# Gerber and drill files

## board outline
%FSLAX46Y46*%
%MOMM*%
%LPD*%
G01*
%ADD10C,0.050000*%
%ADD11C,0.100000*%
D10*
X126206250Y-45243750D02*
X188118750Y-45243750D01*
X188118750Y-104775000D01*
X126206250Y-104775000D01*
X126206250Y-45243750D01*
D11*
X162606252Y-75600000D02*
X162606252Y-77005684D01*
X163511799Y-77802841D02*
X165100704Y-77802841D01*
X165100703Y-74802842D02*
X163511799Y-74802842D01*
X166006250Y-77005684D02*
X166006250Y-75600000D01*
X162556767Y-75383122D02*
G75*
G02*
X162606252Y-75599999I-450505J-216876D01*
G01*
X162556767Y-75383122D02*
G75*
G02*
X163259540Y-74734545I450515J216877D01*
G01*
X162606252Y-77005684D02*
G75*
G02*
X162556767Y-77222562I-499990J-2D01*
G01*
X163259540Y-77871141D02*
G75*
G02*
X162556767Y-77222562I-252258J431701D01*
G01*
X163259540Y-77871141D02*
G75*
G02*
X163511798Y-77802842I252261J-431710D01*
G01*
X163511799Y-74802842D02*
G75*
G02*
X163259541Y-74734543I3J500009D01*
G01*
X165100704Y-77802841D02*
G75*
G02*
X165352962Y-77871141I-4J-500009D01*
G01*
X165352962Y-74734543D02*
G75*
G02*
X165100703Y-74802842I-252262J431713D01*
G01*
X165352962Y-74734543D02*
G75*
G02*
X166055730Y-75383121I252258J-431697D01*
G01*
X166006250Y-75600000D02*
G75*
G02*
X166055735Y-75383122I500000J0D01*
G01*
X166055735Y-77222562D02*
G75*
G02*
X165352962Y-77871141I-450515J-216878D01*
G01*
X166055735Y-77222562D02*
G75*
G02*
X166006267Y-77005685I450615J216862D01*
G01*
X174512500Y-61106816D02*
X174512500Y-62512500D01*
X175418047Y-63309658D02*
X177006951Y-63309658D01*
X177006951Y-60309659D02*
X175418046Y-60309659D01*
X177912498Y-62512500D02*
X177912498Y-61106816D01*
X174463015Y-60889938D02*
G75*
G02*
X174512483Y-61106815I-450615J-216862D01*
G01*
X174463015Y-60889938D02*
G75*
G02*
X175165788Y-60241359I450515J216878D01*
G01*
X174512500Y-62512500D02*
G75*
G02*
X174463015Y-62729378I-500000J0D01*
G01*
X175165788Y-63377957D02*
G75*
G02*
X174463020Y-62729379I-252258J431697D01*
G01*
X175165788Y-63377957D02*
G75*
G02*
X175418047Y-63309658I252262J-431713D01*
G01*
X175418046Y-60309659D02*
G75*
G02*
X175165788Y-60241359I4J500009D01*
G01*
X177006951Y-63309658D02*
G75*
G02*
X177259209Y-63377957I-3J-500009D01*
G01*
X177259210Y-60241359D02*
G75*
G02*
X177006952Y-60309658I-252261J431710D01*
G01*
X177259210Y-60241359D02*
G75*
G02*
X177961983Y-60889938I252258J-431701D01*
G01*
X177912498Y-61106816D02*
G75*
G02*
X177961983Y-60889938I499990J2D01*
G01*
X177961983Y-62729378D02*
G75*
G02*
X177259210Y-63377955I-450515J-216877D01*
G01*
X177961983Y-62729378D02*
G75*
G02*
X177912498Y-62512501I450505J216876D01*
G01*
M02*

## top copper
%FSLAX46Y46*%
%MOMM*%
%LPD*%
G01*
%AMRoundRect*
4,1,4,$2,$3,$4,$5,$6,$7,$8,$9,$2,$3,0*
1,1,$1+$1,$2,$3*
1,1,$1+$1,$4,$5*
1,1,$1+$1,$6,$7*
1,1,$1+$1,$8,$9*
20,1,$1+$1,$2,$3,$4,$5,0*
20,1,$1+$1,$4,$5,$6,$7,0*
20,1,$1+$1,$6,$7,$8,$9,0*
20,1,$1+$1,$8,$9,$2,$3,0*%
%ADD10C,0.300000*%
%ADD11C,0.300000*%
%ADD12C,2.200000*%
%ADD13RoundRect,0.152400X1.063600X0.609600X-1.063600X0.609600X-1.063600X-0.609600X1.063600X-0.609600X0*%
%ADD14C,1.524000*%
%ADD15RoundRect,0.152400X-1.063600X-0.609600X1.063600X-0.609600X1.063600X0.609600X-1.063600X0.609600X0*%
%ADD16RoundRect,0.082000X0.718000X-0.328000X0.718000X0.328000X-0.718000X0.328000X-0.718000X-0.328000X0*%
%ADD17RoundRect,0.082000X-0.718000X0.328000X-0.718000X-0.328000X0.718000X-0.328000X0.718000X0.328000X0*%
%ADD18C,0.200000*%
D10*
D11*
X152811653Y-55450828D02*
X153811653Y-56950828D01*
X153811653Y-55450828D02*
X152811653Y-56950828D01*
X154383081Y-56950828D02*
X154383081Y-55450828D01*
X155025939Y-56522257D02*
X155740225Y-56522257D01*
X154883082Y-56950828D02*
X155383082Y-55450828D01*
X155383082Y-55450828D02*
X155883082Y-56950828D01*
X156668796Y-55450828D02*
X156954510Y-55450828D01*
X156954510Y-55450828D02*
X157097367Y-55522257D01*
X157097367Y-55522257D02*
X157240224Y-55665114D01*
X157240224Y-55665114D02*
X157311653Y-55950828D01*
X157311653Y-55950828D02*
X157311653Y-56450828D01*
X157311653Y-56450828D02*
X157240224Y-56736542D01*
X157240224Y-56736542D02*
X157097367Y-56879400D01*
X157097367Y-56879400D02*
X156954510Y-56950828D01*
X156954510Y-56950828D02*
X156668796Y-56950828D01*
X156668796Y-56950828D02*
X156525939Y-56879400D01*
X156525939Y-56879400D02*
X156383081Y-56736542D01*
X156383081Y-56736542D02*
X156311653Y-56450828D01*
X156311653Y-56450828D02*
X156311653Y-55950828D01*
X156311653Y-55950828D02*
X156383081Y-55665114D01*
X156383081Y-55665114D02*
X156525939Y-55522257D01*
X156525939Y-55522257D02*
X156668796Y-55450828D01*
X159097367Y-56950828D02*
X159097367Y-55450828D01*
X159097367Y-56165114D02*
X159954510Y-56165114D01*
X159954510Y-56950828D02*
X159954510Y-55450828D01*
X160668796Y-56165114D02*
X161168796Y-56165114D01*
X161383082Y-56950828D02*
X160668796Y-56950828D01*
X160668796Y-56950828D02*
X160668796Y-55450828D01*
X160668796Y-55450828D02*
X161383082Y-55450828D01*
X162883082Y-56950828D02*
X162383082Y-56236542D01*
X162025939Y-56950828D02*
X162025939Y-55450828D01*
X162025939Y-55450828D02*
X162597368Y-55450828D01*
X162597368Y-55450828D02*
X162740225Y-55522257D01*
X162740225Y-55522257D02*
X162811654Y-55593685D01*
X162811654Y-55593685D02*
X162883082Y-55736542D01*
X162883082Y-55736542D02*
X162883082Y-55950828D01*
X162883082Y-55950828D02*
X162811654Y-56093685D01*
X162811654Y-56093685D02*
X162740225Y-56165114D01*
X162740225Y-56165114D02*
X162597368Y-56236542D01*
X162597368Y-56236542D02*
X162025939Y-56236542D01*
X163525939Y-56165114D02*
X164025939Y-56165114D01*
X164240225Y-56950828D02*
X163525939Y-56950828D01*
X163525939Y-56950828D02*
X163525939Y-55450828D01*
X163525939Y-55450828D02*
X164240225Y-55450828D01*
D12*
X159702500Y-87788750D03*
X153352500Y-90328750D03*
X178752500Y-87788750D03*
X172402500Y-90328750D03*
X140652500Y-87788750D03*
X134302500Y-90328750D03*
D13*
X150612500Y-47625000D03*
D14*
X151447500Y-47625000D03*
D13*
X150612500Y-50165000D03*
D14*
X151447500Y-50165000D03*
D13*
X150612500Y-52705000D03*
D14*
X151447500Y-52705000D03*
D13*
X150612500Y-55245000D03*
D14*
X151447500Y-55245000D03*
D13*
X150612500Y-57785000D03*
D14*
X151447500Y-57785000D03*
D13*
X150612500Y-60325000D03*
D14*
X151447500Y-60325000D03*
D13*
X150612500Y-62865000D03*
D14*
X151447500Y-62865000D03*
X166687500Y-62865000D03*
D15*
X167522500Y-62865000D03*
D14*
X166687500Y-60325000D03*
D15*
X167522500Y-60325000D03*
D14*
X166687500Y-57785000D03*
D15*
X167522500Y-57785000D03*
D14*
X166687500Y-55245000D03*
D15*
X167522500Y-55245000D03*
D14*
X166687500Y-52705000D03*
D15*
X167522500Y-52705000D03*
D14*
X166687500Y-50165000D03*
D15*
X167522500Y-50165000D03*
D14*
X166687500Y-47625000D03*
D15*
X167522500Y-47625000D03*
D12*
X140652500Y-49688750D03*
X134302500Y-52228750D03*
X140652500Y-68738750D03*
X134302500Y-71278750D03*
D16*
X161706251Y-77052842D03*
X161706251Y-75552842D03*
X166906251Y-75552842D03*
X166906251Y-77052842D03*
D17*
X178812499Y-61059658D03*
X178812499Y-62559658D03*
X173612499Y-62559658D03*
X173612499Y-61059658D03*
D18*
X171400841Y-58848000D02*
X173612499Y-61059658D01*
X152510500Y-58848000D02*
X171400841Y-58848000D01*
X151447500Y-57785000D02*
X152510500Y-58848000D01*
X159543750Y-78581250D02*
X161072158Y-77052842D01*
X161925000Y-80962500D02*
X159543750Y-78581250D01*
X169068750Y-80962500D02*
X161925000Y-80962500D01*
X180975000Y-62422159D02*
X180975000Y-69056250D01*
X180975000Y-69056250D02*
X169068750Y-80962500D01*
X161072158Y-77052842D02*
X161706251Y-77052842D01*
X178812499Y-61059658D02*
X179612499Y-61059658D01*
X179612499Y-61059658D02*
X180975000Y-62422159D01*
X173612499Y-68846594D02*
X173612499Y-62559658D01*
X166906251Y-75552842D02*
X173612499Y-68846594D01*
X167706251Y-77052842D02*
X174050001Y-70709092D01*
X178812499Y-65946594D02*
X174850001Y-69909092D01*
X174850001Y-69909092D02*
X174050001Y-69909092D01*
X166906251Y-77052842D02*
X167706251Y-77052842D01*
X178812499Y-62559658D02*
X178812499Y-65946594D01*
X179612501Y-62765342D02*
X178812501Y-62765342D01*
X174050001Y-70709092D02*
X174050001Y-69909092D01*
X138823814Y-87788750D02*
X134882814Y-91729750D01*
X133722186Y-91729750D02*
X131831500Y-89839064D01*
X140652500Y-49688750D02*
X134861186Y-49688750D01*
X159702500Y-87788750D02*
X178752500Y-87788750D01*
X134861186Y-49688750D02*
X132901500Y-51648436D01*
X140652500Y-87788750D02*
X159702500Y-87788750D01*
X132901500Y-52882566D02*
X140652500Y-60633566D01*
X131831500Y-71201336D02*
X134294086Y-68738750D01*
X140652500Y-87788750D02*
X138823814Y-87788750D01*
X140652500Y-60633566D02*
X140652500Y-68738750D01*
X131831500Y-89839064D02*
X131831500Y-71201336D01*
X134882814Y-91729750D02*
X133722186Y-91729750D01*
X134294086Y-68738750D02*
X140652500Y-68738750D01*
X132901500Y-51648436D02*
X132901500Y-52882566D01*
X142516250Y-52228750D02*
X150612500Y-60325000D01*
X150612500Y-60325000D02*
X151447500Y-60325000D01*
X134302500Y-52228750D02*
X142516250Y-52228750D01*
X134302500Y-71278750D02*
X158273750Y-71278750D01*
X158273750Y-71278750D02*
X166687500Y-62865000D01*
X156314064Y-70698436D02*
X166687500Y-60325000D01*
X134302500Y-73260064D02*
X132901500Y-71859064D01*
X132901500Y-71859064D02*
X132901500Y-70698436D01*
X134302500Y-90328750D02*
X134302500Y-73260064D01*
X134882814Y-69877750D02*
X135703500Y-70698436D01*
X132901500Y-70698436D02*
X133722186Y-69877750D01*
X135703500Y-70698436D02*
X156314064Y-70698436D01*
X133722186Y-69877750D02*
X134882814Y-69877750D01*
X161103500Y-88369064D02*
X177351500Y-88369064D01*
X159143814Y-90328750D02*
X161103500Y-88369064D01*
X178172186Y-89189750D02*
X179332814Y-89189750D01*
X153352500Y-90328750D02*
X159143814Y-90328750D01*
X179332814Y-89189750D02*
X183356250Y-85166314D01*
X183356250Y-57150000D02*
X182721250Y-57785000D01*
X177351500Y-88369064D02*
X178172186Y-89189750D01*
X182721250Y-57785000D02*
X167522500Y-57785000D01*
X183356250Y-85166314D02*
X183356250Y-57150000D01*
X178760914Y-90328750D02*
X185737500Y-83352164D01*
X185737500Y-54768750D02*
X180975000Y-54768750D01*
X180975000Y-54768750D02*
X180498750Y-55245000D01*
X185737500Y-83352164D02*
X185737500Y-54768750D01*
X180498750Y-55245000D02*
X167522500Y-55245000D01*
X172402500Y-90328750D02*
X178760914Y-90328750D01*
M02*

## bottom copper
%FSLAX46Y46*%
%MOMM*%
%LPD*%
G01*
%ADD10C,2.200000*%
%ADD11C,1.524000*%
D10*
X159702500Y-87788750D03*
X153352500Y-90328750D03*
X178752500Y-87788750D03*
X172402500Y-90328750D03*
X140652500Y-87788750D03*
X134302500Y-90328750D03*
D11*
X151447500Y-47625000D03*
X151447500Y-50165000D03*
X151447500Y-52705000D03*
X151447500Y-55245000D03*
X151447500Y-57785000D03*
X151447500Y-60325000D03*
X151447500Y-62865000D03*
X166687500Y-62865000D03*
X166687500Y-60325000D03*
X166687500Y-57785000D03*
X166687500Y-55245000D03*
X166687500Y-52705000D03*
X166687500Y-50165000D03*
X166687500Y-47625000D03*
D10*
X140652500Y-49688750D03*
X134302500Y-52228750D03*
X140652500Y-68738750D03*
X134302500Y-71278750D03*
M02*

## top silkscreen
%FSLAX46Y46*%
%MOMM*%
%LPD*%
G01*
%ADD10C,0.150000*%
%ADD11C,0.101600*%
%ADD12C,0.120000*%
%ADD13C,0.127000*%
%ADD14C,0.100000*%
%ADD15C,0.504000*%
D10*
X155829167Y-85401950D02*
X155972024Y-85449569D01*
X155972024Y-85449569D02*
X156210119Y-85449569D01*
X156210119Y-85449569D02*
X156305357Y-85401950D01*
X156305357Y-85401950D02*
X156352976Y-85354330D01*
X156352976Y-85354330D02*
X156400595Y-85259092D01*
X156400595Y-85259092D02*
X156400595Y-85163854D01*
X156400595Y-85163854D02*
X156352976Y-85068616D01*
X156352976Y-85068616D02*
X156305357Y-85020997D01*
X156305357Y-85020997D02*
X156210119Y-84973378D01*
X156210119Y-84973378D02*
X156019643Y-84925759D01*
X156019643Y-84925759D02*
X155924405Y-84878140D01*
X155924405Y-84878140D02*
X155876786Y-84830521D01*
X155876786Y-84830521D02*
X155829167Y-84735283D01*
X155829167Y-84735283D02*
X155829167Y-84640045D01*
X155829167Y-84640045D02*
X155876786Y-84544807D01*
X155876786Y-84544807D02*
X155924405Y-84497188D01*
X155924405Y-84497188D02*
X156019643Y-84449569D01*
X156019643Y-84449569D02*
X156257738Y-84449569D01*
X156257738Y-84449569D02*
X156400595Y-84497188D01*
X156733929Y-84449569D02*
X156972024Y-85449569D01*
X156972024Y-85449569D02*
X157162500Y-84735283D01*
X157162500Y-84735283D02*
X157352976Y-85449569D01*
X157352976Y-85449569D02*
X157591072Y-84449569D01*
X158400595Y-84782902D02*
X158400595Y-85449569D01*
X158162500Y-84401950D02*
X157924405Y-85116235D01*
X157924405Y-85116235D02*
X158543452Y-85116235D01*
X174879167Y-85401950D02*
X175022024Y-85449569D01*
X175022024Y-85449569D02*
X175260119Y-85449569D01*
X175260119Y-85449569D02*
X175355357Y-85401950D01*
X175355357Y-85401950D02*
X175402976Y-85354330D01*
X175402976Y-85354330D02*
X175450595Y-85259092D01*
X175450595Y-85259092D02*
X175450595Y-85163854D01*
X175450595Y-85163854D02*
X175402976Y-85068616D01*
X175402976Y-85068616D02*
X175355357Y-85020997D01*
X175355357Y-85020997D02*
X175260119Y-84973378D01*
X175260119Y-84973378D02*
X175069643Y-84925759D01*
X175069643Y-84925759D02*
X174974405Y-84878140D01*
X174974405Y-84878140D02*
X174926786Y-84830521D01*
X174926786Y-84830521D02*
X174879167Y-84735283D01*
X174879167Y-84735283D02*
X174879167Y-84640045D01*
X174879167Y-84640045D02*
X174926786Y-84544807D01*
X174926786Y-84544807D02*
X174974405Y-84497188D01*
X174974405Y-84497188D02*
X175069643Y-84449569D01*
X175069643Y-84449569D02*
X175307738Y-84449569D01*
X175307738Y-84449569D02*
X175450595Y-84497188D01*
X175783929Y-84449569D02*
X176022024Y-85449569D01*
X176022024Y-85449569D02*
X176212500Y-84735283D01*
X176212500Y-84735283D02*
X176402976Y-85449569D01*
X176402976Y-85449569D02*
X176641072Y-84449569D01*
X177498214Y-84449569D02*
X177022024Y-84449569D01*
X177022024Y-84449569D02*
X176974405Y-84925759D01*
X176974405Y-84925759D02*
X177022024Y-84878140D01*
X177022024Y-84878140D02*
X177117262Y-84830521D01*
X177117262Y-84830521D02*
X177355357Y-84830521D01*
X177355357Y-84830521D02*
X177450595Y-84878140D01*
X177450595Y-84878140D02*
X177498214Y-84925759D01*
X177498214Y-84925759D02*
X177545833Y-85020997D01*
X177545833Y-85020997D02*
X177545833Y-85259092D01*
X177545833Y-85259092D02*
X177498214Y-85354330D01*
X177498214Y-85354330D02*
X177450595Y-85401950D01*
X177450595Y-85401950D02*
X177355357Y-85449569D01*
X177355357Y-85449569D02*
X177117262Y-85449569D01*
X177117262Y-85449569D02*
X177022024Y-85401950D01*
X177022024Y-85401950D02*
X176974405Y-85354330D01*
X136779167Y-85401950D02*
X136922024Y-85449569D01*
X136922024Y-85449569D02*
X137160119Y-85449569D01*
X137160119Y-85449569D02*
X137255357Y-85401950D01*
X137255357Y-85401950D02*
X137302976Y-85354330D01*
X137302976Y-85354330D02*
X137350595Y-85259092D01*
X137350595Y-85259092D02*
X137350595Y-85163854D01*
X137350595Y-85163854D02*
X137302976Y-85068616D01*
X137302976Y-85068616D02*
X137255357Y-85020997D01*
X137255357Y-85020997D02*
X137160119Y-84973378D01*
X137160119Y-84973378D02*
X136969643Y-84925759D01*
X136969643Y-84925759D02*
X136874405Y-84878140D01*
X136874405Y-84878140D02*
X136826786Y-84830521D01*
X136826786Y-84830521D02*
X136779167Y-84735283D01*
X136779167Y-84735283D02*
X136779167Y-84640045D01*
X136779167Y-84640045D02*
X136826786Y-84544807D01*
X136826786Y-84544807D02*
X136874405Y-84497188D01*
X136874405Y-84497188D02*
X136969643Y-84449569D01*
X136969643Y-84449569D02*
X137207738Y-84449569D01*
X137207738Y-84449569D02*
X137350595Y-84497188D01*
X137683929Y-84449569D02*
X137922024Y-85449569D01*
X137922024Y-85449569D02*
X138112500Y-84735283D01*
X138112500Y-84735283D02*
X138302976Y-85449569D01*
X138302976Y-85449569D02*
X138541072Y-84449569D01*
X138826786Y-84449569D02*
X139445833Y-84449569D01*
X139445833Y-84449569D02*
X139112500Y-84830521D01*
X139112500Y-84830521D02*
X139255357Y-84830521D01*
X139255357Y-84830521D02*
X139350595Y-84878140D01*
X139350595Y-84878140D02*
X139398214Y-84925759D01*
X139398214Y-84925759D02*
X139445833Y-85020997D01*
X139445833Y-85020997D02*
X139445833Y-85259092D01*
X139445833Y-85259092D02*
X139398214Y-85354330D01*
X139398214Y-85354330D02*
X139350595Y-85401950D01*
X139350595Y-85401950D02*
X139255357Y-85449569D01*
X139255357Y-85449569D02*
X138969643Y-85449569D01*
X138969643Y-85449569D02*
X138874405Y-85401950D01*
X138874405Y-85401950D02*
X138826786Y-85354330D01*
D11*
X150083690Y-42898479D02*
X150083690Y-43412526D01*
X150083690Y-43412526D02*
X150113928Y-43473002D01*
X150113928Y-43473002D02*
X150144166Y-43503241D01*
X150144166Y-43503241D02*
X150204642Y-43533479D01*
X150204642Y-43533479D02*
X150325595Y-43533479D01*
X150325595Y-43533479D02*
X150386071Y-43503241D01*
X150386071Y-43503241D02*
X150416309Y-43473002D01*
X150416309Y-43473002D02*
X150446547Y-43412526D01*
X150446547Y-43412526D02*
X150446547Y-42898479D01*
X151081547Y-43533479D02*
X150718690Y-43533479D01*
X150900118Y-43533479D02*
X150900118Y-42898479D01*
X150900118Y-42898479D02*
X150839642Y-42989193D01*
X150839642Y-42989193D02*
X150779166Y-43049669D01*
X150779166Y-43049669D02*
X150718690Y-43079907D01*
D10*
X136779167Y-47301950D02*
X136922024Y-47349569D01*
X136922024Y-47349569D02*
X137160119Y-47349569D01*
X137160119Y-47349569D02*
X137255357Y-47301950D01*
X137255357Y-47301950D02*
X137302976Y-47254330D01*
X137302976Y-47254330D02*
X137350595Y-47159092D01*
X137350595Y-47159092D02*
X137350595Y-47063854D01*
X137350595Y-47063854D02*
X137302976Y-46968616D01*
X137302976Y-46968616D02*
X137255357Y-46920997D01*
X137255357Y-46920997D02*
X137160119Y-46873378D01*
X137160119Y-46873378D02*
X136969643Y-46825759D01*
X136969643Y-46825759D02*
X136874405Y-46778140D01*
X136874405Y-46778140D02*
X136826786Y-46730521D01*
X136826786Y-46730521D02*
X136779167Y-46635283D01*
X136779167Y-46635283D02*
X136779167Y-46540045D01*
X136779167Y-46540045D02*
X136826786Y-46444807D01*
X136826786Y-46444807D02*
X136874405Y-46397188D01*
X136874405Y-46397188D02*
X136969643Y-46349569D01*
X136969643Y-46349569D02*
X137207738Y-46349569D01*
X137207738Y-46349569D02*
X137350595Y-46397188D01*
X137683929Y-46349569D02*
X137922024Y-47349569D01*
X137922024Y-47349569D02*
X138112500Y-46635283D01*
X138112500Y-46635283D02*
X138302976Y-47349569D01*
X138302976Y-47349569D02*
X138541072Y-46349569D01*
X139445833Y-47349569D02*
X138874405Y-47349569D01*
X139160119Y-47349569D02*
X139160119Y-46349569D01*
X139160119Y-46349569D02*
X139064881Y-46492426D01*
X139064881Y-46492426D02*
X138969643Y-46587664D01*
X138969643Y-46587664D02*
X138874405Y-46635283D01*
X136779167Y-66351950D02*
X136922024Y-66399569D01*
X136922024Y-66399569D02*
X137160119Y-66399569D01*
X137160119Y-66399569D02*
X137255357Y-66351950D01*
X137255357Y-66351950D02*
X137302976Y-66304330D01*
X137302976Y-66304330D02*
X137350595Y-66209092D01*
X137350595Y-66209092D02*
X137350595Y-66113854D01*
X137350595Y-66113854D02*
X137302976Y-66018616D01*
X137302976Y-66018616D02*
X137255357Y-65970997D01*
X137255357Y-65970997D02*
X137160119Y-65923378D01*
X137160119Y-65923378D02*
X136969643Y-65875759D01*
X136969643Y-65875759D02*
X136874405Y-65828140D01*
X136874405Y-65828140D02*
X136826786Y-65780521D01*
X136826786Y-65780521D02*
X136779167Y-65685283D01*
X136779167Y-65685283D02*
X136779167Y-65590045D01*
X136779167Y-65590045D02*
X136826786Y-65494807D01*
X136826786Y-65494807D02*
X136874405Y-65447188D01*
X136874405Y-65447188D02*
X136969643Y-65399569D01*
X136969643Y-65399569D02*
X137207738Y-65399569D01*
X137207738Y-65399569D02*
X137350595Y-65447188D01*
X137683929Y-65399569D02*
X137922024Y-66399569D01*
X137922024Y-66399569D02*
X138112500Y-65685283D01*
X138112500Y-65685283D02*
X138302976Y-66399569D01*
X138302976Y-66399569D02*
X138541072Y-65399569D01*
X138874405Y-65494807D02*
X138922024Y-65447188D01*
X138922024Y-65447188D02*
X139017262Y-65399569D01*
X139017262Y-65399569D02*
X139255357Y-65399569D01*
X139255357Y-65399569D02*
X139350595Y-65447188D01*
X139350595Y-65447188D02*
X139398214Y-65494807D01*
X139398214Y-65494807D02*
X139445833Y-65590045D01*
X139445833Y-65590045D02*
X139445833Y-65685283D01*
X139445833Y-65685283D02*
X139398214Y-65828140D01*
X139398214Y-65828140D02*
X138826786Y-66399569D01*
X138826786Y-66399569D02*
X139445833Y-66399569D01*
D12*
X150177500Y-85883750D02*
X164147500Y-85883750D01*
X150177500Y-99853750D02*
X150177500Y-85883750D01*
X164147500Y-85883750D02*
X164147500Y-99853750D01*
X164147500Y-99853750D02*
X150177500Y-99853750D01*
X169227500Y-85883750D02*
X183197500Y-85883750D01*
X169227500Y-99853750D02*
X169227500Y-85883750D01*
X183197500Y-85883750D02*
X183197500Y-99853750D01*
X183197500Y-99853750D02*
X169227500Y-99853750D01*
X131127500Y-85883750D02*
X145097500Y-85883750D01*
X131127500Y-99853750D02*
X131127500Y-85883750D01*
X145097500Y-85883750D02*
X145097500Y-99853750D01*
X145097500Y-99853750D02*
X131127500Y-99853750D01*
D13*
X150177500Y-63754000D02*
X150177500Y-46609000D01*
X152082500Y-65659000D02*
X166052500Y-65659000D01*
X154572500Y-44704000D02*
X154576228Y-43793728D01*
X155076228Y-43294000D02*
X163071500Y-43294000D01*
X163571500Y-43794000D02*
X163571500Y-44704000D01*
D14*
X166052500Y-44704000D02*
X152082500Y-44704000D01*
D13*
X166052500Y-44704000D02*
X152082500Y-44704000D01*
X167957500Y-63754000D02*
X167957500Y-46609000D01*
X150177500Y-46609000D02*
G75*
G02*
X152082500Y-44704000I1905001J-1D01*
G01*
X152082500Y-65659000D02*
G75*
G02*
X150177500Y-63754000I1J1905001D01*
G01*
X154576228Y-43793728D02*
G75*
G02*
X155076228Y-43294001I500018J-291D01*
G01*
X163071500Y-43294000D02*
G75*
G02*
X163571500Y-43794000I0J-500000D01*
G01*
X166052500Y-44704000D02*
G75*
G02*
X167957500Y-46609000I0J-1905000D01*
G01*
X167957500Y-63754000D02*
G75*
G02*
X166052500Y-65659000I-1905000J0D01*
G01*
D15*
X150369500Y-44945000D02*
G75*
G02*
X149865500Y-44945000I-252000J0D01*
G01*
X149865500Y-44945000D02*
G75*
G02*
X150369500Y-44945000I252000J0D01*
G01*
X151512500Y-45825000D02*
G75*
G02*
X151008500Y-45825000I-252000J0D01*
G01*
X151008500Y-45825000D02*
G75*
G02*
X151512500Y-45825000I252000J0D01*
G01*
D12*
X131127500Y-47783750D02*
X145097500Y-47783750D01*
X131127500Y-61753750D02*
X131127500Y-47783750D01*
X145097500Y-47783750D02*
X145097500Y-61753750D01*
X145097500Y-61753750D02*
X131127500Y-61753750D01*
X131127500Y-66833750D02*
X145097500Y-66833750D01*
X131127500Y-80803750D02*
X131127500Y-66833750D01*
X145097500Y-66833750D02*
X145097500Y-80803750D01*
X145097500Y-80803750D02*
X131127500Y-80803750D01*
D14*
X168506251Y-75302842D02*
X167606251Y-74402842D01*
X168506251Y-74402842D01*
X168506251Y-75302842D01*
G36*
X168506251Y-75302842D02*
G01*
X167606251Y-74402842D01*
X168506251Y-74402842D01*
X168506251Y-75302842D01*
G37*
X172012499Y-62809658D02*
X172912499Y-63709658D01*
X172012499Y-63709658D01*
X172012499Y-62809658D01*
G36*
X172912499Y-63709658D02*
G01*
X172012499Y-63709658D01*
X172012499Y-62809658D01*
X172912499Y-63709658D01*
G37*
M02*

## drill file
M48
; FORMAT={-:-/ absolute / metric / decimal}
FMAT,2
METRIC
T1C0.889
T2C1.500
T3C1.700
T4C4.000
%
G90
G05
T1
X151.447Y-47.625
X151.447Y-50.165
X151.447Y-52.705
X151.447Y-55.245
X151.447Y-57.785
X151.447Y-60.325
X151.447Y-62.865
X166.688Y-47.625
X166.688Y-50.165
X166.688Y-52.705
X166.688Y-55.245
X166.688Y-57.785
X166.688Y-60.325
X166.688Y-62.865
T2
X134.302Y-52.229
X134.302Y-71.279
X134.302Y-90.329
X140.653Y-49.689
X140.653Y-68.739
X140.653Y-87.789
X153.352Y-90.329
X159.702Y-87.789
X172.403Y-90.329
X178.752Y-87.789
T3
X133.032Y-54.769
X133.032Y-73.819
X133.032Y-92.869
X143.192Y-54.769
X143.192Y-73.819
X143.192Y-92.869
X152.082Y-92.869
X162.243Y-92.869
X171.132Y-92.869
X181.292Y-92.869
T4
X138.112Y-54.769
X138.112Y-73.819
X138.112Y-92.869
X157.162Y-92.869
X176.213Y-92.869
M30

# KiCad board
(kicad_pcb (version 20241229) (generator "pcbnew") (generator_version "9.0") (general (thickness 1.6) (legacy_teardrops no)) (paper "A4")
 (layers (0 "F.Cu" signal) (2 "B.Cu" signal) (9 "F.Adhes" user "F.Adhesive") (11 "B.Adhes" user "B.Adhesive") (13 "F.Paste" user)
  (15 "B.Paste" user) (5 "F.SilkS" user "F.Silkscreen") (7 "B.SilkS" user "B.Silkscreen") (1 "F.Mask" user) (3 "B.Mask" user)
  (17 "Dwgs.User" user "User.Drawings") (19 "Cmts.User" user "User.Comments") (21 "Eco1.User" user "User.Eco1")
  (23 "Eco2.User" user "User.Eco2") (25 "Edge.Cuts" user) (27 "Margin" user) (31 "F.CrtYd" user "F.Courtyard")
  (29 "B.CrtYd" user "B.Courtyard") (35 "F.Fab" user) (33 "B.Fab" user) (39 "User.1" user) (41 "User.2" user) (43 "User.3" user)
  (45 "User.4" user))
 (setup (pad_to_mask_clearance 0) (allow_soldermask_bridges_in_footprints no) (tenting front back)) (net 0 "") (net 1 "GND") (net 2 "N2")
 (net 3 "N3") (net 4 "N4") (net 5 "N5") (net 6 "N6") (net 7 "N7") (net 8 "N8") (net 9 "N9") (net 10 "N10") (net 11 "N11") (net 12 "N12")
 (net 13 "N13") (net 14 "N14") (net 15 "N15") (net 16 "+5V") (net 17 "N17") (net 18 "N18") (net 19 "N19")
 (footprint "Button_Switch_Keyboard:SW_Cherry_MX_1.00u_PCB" (layer "F.Cu") (at 159.7025 87.78875)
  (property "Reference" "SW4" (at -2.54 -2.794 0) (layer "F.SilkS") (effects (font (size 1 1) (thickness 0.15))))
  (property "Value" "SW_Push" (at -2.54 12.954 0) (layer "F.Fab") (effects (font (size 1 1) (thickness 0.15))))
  (fp_line (start -9.525 -1.905) (end 4.445 -1.905) (stroke (width 0.12) (type solid)) (layer "F.SilkS"))
  (fp_line (start -9.525 12.065) (end -9.525 -1.905) (stroke (width 0.12) (type solid)) (layer "F.SilkS"))
  (fp_line (start 4.445 -1.905) (end 4.445 12.065) (stroke (width 0.12) (type solid)) (layer "F.SilkS"))
  (fp_line (start 4.445 12.065) (end -9.525 12.065) (stroke (width 0.12) (type solid)) (layer "F.SilkS"))
  (pad "" np_thru_hole circle (at -7.62 5.08) (size 1.7 1.7) (drill 1.7) (layers "*.Cu" "*.Mask"))
  (pad "" np_thru_hole circle (at -2.54 5.08) (size 4 4) (drill 4) (layers "*.Cu" "*.Mask"))
  (pad "" np_thru_hole circle (at 2.54 5.08) (size 1.7 1.7) (drill 1.7) (layers "*.Cu" "*.Mask"))
  (pad "1" thru_hole circle (at 0 0) (size 2.2 2.2) (drill 1.5) (layers "*.Cu" "*.Mask") (remove_unused_layers no) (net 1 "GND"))
  (pad "2" thru_hole circle (at -6.35 2.54) (size 2.2 2.2) (drill 1.5) (layers "*.Cu" "*.Mask") (remove_unused_layers no) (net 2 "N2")))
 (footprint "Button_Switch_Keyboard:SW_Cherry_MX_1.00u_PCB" (layer "F.Cu") (at 178.7525 87.78875)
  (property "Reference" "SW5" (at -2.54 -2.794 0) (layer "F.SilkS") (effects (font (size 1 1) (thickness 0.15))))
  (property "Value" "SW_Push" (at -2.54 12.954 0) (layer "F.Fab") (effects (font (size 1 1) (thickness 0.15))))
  (fp_line (start -9.525 -1.905) (end 4.445 -1.905) (stroke (width 0.12) (type solid)) (layer "F.SilkS"))
  (fp_line (start -9.525 12.065) (end -9.525 -1.905) (stroke (width 0.12) (type solid)) (layer "F.SilkS"))
  (fp_line (start 4.445 -1.905) (end 4.445 12.065) (stroke (width 0.12) (type solid)) (layer "F.SilkS"))
  (fp_line (start 4.445 12.065) (end -9.525 12.065) (stroke (width 0.12) (type solid)) (layer "F.SilkS"))
  (pad "" np_thru_hole circle (at -7.62 5.08) (size 1.7 1.7) (drill 1.7) (layers "*.Cu" "*.Mask"))
  (pad "" np_thru_hole circle (at -2.54 5.08) (size 4 4) (drill 4) (layers "*.Cu" "*.Mask"))
  (pad "" np_thru_hole circle (at 2.54 5.08) (size 1.7 1.7) (drill 1.7) (layers "*.Cu" "*.Mask"))
  (pad "1" thru_hole circle (at 0 0) (size 2.2 2.2) (drill 1.5) (layers "*.Cu" "*.Mask") (remove_unused_layers no) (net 1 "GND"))
  (pad "2" thru_hole circle (at -6.35 2.54) (size 2.2 2.2) (drill 1.5) (layers "*.Cu" "*.Mask") (remove_unused_layers no) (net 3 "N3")))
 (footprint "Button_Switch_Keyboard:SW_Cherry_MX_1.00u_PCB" (layer "F.Cu") (at 140.6525 87.78875)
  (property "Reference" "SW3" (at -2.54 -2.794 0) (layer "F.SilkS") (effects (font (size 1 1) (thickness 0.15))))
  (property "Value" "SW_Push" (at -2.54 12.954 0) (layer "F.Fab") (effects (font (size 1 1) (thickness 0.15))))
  (fp_line (start -9.525 -1.905) (end 4.445 -1.905) (stroke (width 0.12) (type solid)) (layer "F.SilkS"))
  (fp_line (start -9.525 12.065) (end -9.525 -1.905) (stroke (width 0.12) (type solid)) (layer "F.SilkS"))
  (fp_line (start 4.445 -1.905) (end 4.445 12.065) (stroke (width 0.12) (type solid)) (layer "F.SilkS"))
  (fp_line (start 4.445 12.065) (end -9.525 12.065) (stroke (width 0.12) (type solid)) (layer "F.SilkS"))
  (pad "" np_thru_hole circle (at -7.62 5.08) (size 1.7 1.7) (drill 1.7) (layers "*.Cu" "*.Mask"))
  (pad "" np_thru_hole circle (at -2.54 5.08) (size 4 4) (drill 4) (layers "*.Cu" "*.Mask"))
  (pad "" np_thru_hole circle (at 2.54 5.08) (size 1.7 1.7) (drill 1.7) (layers "*.Cu" "*.Mask"))
  (pad "1" thru_hole circle (at 0 0) (size 2.2 2.2) (drill 1.5) (layers "*.Cu" "*.Mask") (remove_unused_layers no) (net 1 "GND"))
  (pad "2" thru_hole circle (at -6.35 2.54) (size 2.2 2.2) (drill 1.5) (layers "*.Cu" "*.Mask") (remove_unused_layers no) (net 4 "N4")))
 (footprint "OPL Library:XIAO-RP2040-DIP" (layer "F.Cu") (at 159.0675 55.245)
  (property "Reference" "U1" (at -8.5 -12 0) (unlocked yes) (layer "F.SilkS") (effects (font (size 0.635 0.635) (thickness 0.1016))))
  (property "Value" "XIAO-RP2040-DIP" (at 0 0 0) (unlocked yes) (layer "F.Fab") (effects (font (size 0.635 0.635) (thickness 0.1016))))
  (fp_line (start -8.89 8.509) (end -8.89 -8.636) (stroke (width 0.127) (type solid)) (layer "F.SilkS"))
  (fp_line (start -6.985 10.414) (end 6.985 10.414) (stroke (width 0.127) (type solid)) (layer "F.SilkS"))
  (fp_line (start -4.495 -10.541) (end -4.491272 -11.451272) (stroke (width 0.127) (type solid)) (layer "F.SilkS"))
  (fp_line (start -3.991272 -11.951) (end 4.004 -11.951) (stroke (width 0.127) (type solid)) (layer "F.SilkS"))
  (fp_line (start 4.504 -11.451) (end 4.504 -10.541) (stroke (width 0.127) (type solid)) (layer "F.SilkS"))
  (fp_line (start 6.985 -10.541) (end -6.985 -10.541) (stroke (width 0.1) (type solid)) (layer "F.SilkS"))
  (fp_line (start 6.985 -10.541) (end -6.985 -10.541) (stroke (width 0.127) (type solid)) (layer "F.SilkS"))
  (fp_line (start 8.89 8.509) (end 8.89 -8.636) (stroke (width 0.127) (type solid)) (layer "F.SilkS"))
  (fp_arc (start -8.89 -8.636) (mid -8.332038 -9.983038) (end -6.985 -10.541) (stroke (width 0.127) (type solid)) (layer "F.SilkS"))
  (fp_arc (start -6.985 10.414) (mid -8.332038 9.856038) (end -8.89 8.509) (stroke (width 0.127) (type solid)) (layer "F.SilkS"))
  (fp_arc (start -4.491272 -11.451272) (mid -4.344728 -11.80464) (end -3.991272 -11.951) (stroke (width 0.127) (type default))
   (layer "F.SilkS"))
  (fp_arc (start 4.004 -11.951) (mid 4.357553 -11.804553) (end 4.504 -11.451) (stroke (width 0.127) (type default)) (layer "F.SilkS"))
  (fp_arc (start 6.985 -10.541) (mid 8.332038 -9.983038) (end 8.89 -8.636) (stroke (width 0.127) (type solid)) (layer "F.SilkS"))
  (fp_arc (start 8.89 8.509) (mid 8.332038 9.856038) (end 6.985 10.414) (stroke (width 0.127) (type solid)) (layer "F.SilkS"))
  (fp_circle (center -8.95 -10.3) (end -8.95 -10.554) (stroke (width 0.5) (type solid)) (fill yes) (layer "F.SilkS"))
  (fp_circle (center -7.807 -9.42) (end -7.807 -9.674) (stroke (width 0.5) (type solid)) (fill yes) (layer "F.SilkS"))
  (pad "1" smd roundrect (at -8.455 -7.62 180) (size 2.432 1.524) (layers "F.Cu" "F.Mask") (roundrect_rratio 0.1) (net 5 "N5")
   (thermal_bridge_angle 45))
  (pad "1" thru_hole circle (at -7.62 -7.62 180) (size 1.524 1.524) (drill 0.889) (layers "*.Cu" "*.Mask") (remove_unused_layers no)
   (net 5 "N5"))
  (pad "2" smd roundrect (at -8.455 -5.08 180) (size 2.432 1.524) (layers "F.Cu" "F.Mask") (roundrect_rratio 0.1) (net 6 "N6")
   (thermal_bridge_angle 45))
  (pad "2" thru_hole circle (at -7.62 -5.08 180) (size 1.524 1.524) (drill 0.889) (layers "*.Cu" "*.Mask") (remove_unused_layers no)
   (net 6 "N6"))
  (pad "3" smd roundrect (at -8.455 -2.54 180) (size 2.432 1.524) (layers "F.Cu" "F.Mask") (roundrect_rratio 0.1) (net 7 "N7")
   (thermal_bridge_angle 45))
  (pad "3" thru_hole circle (at -7.62 -2.54 180) (size 1.524 1.524) (drill 0.889) (layers "*.Cu" "*.Mask") (remove_unused_layers no)
   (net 7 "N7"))
  (pad "4" smd roundrect (at -8.455 0 180) (size 2.432 1.524) (layers "F.Cu" "F.Mask") (roundrect_rratio 0.1) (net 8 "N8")
   (thermal_bridge_angle 45))
  (pad "4" thru_hole circle (at -7.62 0 180) (size 1.524 1.524) (drill 0.889) (layers "*.Cu" "*.Mask") (remove_unused_layers no)
   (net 8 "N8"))
  (pad "5" smd roundrect (at -8.455 2.54 180) (size 2.432 1.524) (layers "F.Cu" "F.Mask") (roundrect_rratio 0.1) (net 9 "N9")
   (thermal_bridge_angle 45))
  (pad "5" thru_hole circle (at -7.62 2.54 180) (size 1.524 1.524) (drill 0.889) (layers "*.Cu" "*.Mask") (remove_unused_layers no)
   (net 9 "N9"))
  (pad "6" smd roundrect (at -8.455 5.08 180) (size 2.432 1.524) (layers "F.Cu" "F.Mask") (roundrect_rratio 0.1) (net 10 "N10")
   (thermal_bridge_angle 45))
  (pad "6" thru_hole circle (at -7.62 5.08 180) (size 1.524 1.524) (drill 0.889) (layers "*.Cu" "*.Mask") (remove_unused_layers no)
   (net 10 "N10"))
  (pad "7" smd roundrect (at -8.455 7.62 180) (size 2.432 1.524) (layers "F.Cu" "F.Mask") (roundrect_rratio 0.1) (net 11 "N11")
   (thermal_bridge_angle 45))
  (pad "7" thru_hole circle (at -7.62 7.62 180) (size 1.524 1.524) (drill 0.889) (layers "*.Cu" "*.Mask") (remove_unused_layers no)
   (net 11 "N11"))
  (pad "8" thru_hole circle (at 7.62 7.62) (size 1.524 1.524) (drill 0.889) (layers "*.Cu" "*.Mask") (remove_unused_layers no)
   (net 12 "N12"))
  (pad "8" smd roundrect (at 8.455 7.62) (size 2.432 1.524) (layers "F.Cu" "F.Mask") (roundrect_rratio 0.1) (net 12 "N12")
   (thermal_bridge_angle 45))
  (pad "9" thru_hole circle (at 7.62 5.08) (size 1.524 1.524) (drill 0.889) (layers "*.Cu" "*.Mask") (remove_unused_layers no) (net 4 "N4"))
  (pad "9" smd roundrect (at 8.455 5.08) (size 2.432 1.524) (layers "F.Cu" "F.Mask") (roundrect_rratio 0.1) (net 4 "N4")
   (thermal_bridge_angle 45))
  (pad "10" thru_hole circle (at 7.62 2.54) (size 1.524 1.524) (drill 0.889) (layers "*.Cu" "*.Mask") (remove_unused_layers no) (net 2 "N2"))
  (pad "10" smd roundrect (at 8.455 2.54) (size 2.432 1.524) (layers "F.Cu" "F.Mask") (roundrect_rratio 0.1) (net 2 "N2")
   (thermal_bridge_angle 45))
  (pad "11" thru_hole circle (at 7.62 0) (size 1.524 1.524) (drill 0.889) (layers "*.Cu" "*.Mask") (remove_unused_layers no) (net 3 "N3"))
  (pad "11" smd roundrect (at 8.455 0) (size 2.432 1.524) (layers "F.Cu" "F.Mask") (roundrect_rratio 0.1) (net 3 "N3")
   (thermal_bridge_angle 45))
  (pad "12" thru_hole circle (at 7.62 -2.54) (size 1.524 1.524) (drill 0.889) (layers "*.Cu" "*.Mask") (remove_unused_layers no)
   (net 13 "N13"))
  (pad "12" smd roundrect (at 8.455 -2.54) (size 2.432 1.524) (layers "F.Cu" "F.Mask") (roundrect_rratio 0.1) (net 13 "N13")
   (thermal_bridge_angle 45))
  (pad "13" thru_hole circle (at 7.62 -5.08) (size 1.524 1.524) (drill 0.889) (layers "*.Cu" "*.Mask") (remove_unused_layers no)
   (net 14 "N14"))
  (pad "13" smd roundrect (at 8.455 -5.08) (size 2.432 1.524) (layers "F.Cu" "F.Mask") (roundrect_rratio 0.1) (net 14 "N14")
   (thermal_bridge_angle 45))
  (pad "14" thru_hole circle (at 7.62 -7.62) (size 1.524 1.524) (drill 0.889) (layers "*.Cu" "*.Mask") (remove_unused_layers no)
   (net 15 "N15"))
  (pad "14" smd roundrect (at 8.455 -7.62) (size 2.432 1.524) (layers "F.Cu" "F.Mask") (roundrect_rratio 0.1) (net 15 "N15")
   (thermal_bridge_angle 45)))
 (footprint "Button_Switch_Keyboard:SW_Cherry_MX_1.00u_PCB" (layer "F.Cu") (at 140.6525 49.68875)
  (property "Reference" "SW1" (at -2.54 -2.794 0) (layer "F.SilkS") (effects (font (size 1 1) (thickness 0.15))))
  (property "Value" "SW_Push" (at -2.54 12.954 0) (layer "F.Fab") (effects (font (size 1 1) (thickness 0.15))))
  (fp_line (start -9.525 -1.905) (end 4.445 -1.905) (stroke (width 0.12) (type solid)) (layer "F.SilkS"))
  (fp_line (start -9.525 12.065) (end -9.525 -1.905) (stroke (width 0.12) (type solid)) (layer "F.SilkS"))
  (fp_line (start 4.445 -1.905) (end 4.445 12.065) (stroke (width 0.12) (type solid)) (layer "F.SilkS"))
  (fp_line (start 4.445 12.065) (end -9.525 12.065) (stroke (width 0.12) (type solid)) (layer "F.SilkS"))
  (pad "" np_thru_hole circle (at -7.62 5.08) (size 1.7 1.7) (drill 1.7) (layers "*.Cu" "*.Mask"))
  (pad "" np_thru_hole circle (at -2.54 5.08) (size 4 4) (drill 4) (layers "*.Cu" "*.Mask"))
  (pad "" np_thru_hole circle (at 2.54 5.08) (size 1.7 1.7) (drill 1.7) (layers "*.Cu" "*.Mask"))
  (pad "1" thru_hole circle (at 0 0) (size 2.2 2.2) (drill 1.5) (layers "*.Cu" "*.Mask") (remove_unused_layers no) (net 1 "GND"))
  (pad "2" thru_hole circle (at -6.35 2.54) (size 2.2 2.2) (drill 1.5) (layers "*.Cu" "*.Mask") (remove_unused_layers no) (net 10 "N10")))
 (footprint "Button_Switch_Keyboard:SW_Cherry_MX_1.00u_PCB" (layer "F.Cu") (at 140.6525 68.73875)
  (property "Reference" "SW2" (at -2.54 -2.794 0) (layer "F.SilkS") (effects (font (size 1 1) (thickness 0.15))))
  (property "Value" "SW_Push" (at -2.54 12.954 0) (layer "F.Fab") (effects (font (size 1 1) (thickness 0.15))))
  (fp_line (start -9.525 -1.905) (end 4.445 -1.905) (stroke (width 0.12) (type solid)) (layer "F.SilkS"))
  (fp_line (start -9.525 12.065) (end -9.525 -1.905) (stroke (width 0.12) (type solid)) (layer "F.SilkS"))
  (fp_line (start 4.445 -1.905) (end 4.445 12.065) (stroke (width 0.12) (type solid)) (layer "F.SilkS"))
  (fp_line (start 4.445 12.065) (end -9.525 12.065) (stroke (width 0.12) (type solid)) (layer "F.SilkS"))
  (pad "" np_thru_hole circle (at -7.62 5.08) (size 1.7 1.7) (drill 1.7) (layers "*.Cu" "*.Mask"))
  (pad "" np_thru_hole circle (at -2.54 5.08) (size 4 4) (drill 4) (layers "*.Cu" "*.Mask"))
  (pad "" np_thru_hole circle (at 2.54 5.08) (size 1.7 1.7) (drill 1.7) (layers "*.Cu" "*.Mask"))
  (pad "1" thru_hole circle (at 0 0) (size 2.2 2.2) (drill 1.5) (layers "*.Cu" "*.Mask") (remove_unused_layers no) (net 1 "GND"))
  (pad "2" thru_hole circle (at -6.35 2.54) (size 2.2 2.2) (drill 1.5) (layers "*.Cu" "*.Mask") (remove_unused_layers no) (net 12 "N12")))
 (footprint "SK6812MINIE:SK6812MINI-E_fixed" (layer "B.Cu") (at 164.30625 76.2)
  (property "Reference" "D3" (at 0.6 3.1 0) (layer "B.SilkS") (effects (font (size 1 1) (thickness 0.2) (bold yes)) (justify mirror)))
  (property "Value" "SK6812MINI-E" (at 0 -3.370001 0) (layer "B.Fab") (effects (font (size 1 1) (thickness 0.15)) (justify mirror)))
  (fp_poly
   (pts (xy 4.200001 -0.897158) (xy 3.300001 -1.797158) (xy 4.200001 -1.797158)) (stroke (width 0.1) (type solid)) (fill yes)
   (layer "F.SilkS"))
  (fp_line (start -1.699998 -0.6) (end -1.699998 0.805684) (stroke (width 0.1) (type solid)) (layer "Edge.Cuts"))
  (fp_line (start -0.794451 1.602841) (end 0.794454 1.602841) (stroke (width 0.1) (type solid)) (layer "Edge.Cuts"))
  (fp_line (start 0.794453 -1.397158) (end -0.794451 -1.397158) (stroke (width 0.1) (type solid)) (layer "Edge.Cuts"))
  (fp_line (start 1.7 0.805684) (end 1.7 -0.6) (stroke (width 0.1) (type solid)) (layer "Edge.Cuts"))
  (fp_arc (start -1.749483 -0.816878) (mid -1.712526 -0.711226) (end -1.699998 -0.600001) (stroke (width 0.1) (type solid))
   (layer "Edge.Cuts"))
  (fp_arc (start -1.749483 -0.816878) (mid -1.638069 -1.401192) (end -1.04671 -1.465455) (stroke (width 0.1) (type solid))
   (layer "Edge.Cuts"))
  (fp_arc (start -1.699998 0.805684) (mid -1.712526 0.91691) (end -1.749483 1.022562) (stroke (width 0.1) (type solid)) (layer "Edge.Cuts"))
  (fp_arc (start -1.04671 1.671141) (mid -1.63807 1.606877) (end -1.749483 1.022562) (stroke (width 0.1) (type solid)) (layer "Edge.Cuts"))
  (fp_arc (start -1.04671 1.671141) (mid -0.925122 1.620219) (end -0.794452 1.602842) (stroke (width 0.1) (type solid)) (layer "Edge.Cuts"))
  (fp_arc (start -0.794451 -1.397158) (mid -0.925121 -1.414535) (end -1.046709 -1.465457) (stroke (width 0.1) (type solid))
   (layer "Edge.Cuts"))
  (fp_arc (start 0.794454 1.602841) (mid 0.925124 1.620218) (end 1.046712 1.67114) (stroke (width 0.1) (type solid)) (layer "Edge.Cuts"))
  (fp_arc (start 1.046712 -1.465457) (mid 0.925124 -1.414535) (end 0.794453 -1.397158) (stroke (width 0.1) (type solid)) (layer "Edge.Cuts"))
  (fp_arc (start 1.046712 -1.465457) (mid 1.638073 -1.401193) (end 1.749485 -0.816877) (stroke (width 0.1) (type solid)) (layer "Edge.Cuts"))
  (fp_arc (start 1.7 -0.6) (mid 1.712528 -0.711226) (end 1.749485 -0.816878) (stroke (width 0.1) (type solid)) (layer "Edge.Cuts"))
  (fp_arc (start 1.749485 1.022562) (mid 1.638072 1.606877) (end 1.046712 1.67114) (stroke (width 0.1) (type solid)) (layer "Edge.Cuts"))
  (fp_arc (start 1.749485 1.022562) (mid 1.712532 0.91691) (end 1.7 0.805685) (stroke (width 0.1) (type solid)) (layer "Edge.Cuts"))
  (pad "1" smd roundrect (at -2.599999 0.852842 90) (size 0.82 1.6) (layers "F.Cu" "F.Mask" "F.Paste") (roundrect_rratio 0.1) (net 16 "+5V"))
  (pad "2" smd roundrect (at -2.599999 -0.647158 90) (size 0.82 1.6) (layers "F.Cu" "F.Mask" "F.Paste") (roundrect_rratio 0.1)
   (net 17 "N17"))
  (pad "3" smd roundrect (at 2.600001 -0.647158 90) (size 0.82 1.6) (layers "F.Cu" "F.Mask" "F.Paste") (roundrect_rratio 0.1) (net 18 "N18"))
  (pad "4" smd roundrect (at 2.600001 0.852842 90) (size 0.82 1.6) (layers "F.Cu" "F.Mask" "F.Paste") (roundrect_rratio 0.1) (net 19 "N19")))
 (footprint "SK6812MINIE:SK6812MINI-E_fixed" (layer "B.Cu") (at 176.2125 61.9125 180)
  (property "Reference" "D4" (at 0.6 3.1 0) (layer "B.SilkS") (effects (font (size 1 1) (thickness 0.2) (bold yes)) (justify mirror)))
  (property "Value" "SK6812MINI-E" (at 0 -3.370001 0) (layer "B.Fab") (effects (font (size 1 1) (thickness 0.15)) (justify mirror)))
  (fp_poly
   (pts (xy 4.200001 -0.897158) (xy 3.300001 -1.797158) (xy 4.200001 -1.797158)) (stroke (width 0.1) (type solid)) (fill yes)
   (layer "F.SilkS"))
  (fp_line (start 1.7 0.805684) (end 1.7 -0.6) (stroke (width 0.1) (type solid)) (layer "Edge.Cuts"))
  (fp_line (start 0.794453 -1.397158) (end -0.794451 -1.397158) (stroke (width 0.1) (type solid)) (layer "Edge.Cuts"))
  (fp_line (start -0.794451 1.602841) (end 0.794454 1.602841) (stroke (width 0.1) (type solid)) (layer "Edge.Cuts"))
  (fp_line (start -1.699998 -0.6) (end -1.699998 0.805684) (stroke (width 0.1) (type solid)) (layer "Edge.Cuts"))
  (fp_arc (start 1.749485 1.022562) (mid 1.712532 0.91691) (end 1.7 0.805685) (stroke (width 0.1) (type solid)) (layer "Edge.Cuts"))
  (fp_arc (start 1.749485 1.022562) (mid 1.638072 1.606877) (end 1.046712 1.67114) (stroke (width 0.1) (type solid)) (layer "Edge.Cuts"))
  (fp_arc (start 1.7 -0.6) (mid 1.712528 -0.711226) (end 1.749485 -0.816878) (stroke (width 0.1) (type solid)) (layer "Edge.Cuts"))
  (fp_arc (start 1.046712 -1.465457) (mid 1.638073 -1.401193) (end 1.749485 -0.816877) (stroke (width 0.1) (type solid)) (layer "Edge.Cuts"))
  (fp_arc (start 1.046712 -1.465457) (mid 0.925124 -1.414535) (end 0.794453 -1.397158) (stroke (width 0.1) (type solid)) (layer "Edge.Cuts"))
  (fp_arc (start 0.794454 1.602841) (mid 0.925124 1.620218) (end 1.046712 1.67114) (stroke (width 0.1) (type solid)) (layer "Edge.Cuts"))
  (fp_arc (start -0.794451 -1.397158) (mid -0.925121 -1.414535) (end -1.046709 -1.465457) (stroke (width 0.1) (type solid))
   (layer "Edge.Cuts"))
  (fp_arc (start -1.04671 1.671141) (mid -0.925122 1.620219) (end -0.794452 1.602842) (stroke (width 0.1) (type solid)) (layer "Edge.Cuts"))
  (fp_arc (start -1.04671 1.671141) (mid -1.63807 1.606877) (end -1.749483 1.022562) (stroke (width 0.1) (type solid)) (layer "Edge.Cuts"))
  (fp_arc (start -1.699998 0.805684) (mid -1.712526 0.91691) (end -1.749483 1.022562) (stroke (width 0.1) (type solid)) (layer "Edge.Cuts"))
  (fp_arc (start -1.749483 -0.816878) (mid -1.638069 -1.401192) (end -1.04671 -1.465455) (stroke (width 0.1) (type solid))
   (layer "Edge.Cuts"))
  (fp_arc (start -1.749483 -0.816878) (mid -1.712526 -0.711226) (end -1.699998 -0.600001) (stroke (width 0.1) (type solid))
   (layer "Edge.Cuts"))
  (pad "1" smd roundrect (at -2.599999 0.852842 270) (size 0.82 1.6) (layers "F.Cu" "F.Mask" "F.Paste") (roundrect_rratio 0.1)
   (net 16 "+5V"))
  (pad "2" smd roundrect (at -2.599999 -0.647158 270) (size 0.82 1.6) (layers "F.Cu" "F.Mask" "F.Paste") (roundrect_rratio 0.1)
   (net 19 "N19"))
  (pad "3" smd roundrect (at 2.600001 -0.647158 270) (size 0.82 1.6) (layers "F.Cu" "F.Mask" "F.Paste") (roundrect_rratio 0.1)
   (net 18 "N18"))
  (pad "4" smd roundrect (at 2.600001 0.852842 270) (size 0.82 1.6) (layers "F.Cu" "F.Mask" "F.Paste") (roundrect_rratio 0.1) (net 9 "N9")))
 (gr_rect (start 126.20625 45.24375) (end 188.11875 104.775) (stroke (width 0.05) (type default)) (fill no) (layer "Edge.Cuts"))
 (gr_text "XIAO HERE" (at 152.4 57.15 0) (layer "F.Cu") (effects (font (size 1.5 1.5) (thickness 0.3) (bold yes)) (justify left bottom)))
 (segment (start 171.400841 58.848) (end 173.612499 61.059658) (width 0.2) (layer "F.Cu") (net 9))
 (segment (start 152.5105 58.848) (end 171.400841 58.848) (width 0.2) (layer "F.Cu") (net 9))
 (segment (start 151.4475 57.785) (end 152.5105 58.848) (width 0.2) (layer "F.Cu") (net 9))
 (segment (start 159.54375 78.58125) (end 161.072158 77.052842) (width 0.2) (layer "F.Cu") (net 16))
 (segment (start 161.925 80.9625) (end 159.54375 78.58125) (width 0.2) (layer "F.Cu") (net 16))
 (segment (start 169.06875 80.9625) (end 161.925 80.9625) (width 0.2) (layer "F.Cu") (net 16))
 (segment (start 180.975 62.422159) (end 180.975 69.05625) (width 0.2) (layer "F.Cu") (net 16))
 (segment (start 180.975 69.05625) (end 169.06875 80.9625) (width 0.2) (layer "F.Cu") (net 16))
 (segment (start 161.072158 77.052842) (end 161.706251 77.052842) (width 0.2) (layer "F.Cu") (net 16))
 (segment (start 178.812499 61.059658) (end 179.612499 61.059658) (width 0.2) (layer "F.Cu") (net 16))
 (segment (start 179.612499 61.059658) (end 180.975 62.422159) (width 0.2) (layer "F.Cu") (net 16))
 (segment (start 173.612499 68.846594) (end 173.612499 62.559658) (width 0.2) (layer "F.Cu") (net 18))
 (segment (start 166.906251 75.552842) (end 173.612499 68.846594) (width 0.2) (layer "F.Cu") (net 18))
 (segment (start 167.706251 77.052842) (end 174.050001 70.709092) (width 0.2) (layer "F.Cu") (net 19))
 (segment (start 178.812499 65.946594) (end 174.850001 69.909092) (width 0.2) (layer "F.Cu") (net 19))
 (segment (start 174.850001 69.909092) (end 174.050001 69.909092) (width 0.2) (layer "F.Cu") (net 19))
 (segment (start 166.906251 77.052842) (end 167.706251 77.052842) (width 0.2) (layer "F.Cu") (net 19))
 (segment (start 178.812499 62.559658) (end 178.812499 65.946594) (width 0.2) (layer "F.Cu") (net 19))
 (segment (start 179.612501 62.765342) (end 178.812501 62.765342) (width 0.2) (layer "F.Cu") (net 19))
 (segment (start 174.050001 70.709092) (end 174.050001 69.909092) (width 0.2) (layer "F.Cu") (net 19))
 (segment (start 138.823814 87.78875) (end 134.882814 91.72975) (width 0.2) (layer "F.Cu") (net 1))
 (segment (start 133.722186 91.72975) (end 131.8315 89.839064) (width 0.2) (layer "F.Cu") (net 1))
 (segment (start 140.6525 49.68875) (end 134.861186 49.68875) (width 0.2) (layer "F.Cu") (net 1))
 (segment (start 159.7025 87.78875) (end 178.7525 87.78875) (width 0.2) (layer "F.Cu") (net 1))
 (segment (start 134.861186 49.68875) (end 132.9015 51.648436) (width 0.2) (layer "F.Cu") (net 1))
 (segment (start 140.6525 87.78875) (end 159.7025 87.78875) (width 0.2) (layer "F.Cu") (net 1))
 (segment (start 132.9015 52.882566) (end 140.6525 60.633566) (width 0.2) (layer "F.Cu") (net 1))
 (segment (start 131.8315 71.201336) (end 134.294086 68.73875) (width 0.2) (layer "F.Cu") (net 1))
 (segment (start 140.6525 87.78875) (end 138.823814 87.78875) (width 0.2) (layer "F.Cu") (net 1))
 (segment (start 140.6525 60.633566) (end 140.6525 68.73875) (width 0.2) (layer "F.Cu") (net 1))
 (segment (start 131.8315 89.839064) (end 131.8315 71.201336) (width 0.2) (layer "F.Cu") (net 1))
 (segment (start 134.882814 91.72975) (end 133.722186 91.72975) (width 0.2) (layer "F.Cu") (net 1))
 (segment (start 134.294086 68.73875) (end 140.6525 68.73875) (width 0.2) (layer "F.Cu") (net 1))
 (segment (start 132.9015 51.648436) (end 132.9015 52.882566) (width 0.2) (layer "F.Cu") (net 1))
 (segment (start 142.51625 52.22875) (end 150.6125 60.325) (width 0.2) (layer "F.Cu") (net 10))
 (segment (start 150.6125 60.325) (end 151.4475 60.325) (width 0.2) (layer "F.Cu") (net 10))
 (segment (start 134.3025 52.22875) (end 142.51625 52.22875) (width 0.2) (layer "F.Cu") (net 10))
 (segment (start 134.3025 71.27875) (end 158.27375 71.27875) (width 0.2) (layer "F.Cu") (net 12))
 (segment (start 158.27375 71.27875) (end 166.6875 62.865) (width 0.2) (layer "F.Cu") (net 12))
 (segment (start 156.314064 70.698436) (end 166.6875 60.325) (width 0.2) (layer "F.Cu") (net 4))
 (segment (start 134.3025 73.260064) (end 132.9015 71.859064) (width 0.2) (layer "F.Cu") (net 4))
 (segment (start 132.9015 71.859064) (end 132.9015 70.698436) (width 0.2) (layer "F.Cu") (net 4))
 (segment (start 134.3025 90.32875) (end 134.3025 73.260064) (width 0.2) (layer "F.Cu") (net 4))
 (segment (start 134.882814 69.87775) (end 135.7035 70.698436) (width 0.2) (layer "F.Cu") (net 4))
 (segment (start 132.9015 70.698436) (end 133.722186 69.87775) (width 0.2) (layer "F.Cu") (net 4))
 (segment (start 135.7035 70.698436) (end 156.314064 70.698436) (width 0.2) (layer "F.Cu") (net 4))
 (segment (start 133.722186 69.87775) (end 134.882814 69.87775) (width 0.2) (layer "F.Cu") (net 4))
 (segment (start 161.1035 88.369064) (end 177.3515 88.369064) (width 0.2) (layer "F.Cu") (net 2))
 (segment (start 159.143814 90.32875) (end 161.1035 88.369064) (width 0.2) (layer "F.Cu") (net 2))
 (segment (start 178.172186 89.18975) (end 179.332814 89.18975) (width 0.2) (layer "F.Cu") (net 2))
 (segment (start 153.3525 90.32875) (end 159.143814 90.32875) (width 0.2) (layer "F.Cu") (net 2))
 (segment (start 179.332814 89.18975) (end 183.35625 85.166314) (width 0.2) (layer "F.Cu") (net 2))
 (segment (start 183.35625 57.15) (end 182.72125 57.785) (width 0.2) (layer "F.Cu") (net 2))
 (segment (start 177.3515 88.369064) (end 178.172186 89.18975) (width 0.2) (layer "F.Cu") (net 2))
 (segment (start 182.72125 57.785) (end 167.5225 57.785) (width 0.2) (layer "F.Cu") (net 2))
 (segment (start 183.35625 85.166314) (end 183.35625 57.15) (width 0.2) (layer "F.Cu") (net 2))
 (segment (start 178.760914 90.32875) (end 185.7375 83.352164) (width 0.2) (layer "F.Cu") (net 3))
 (segment (start 185.7375 54.76875) (end 180.975 54.76875) (width 0.2) (layer "F.Cu") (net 3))
 (segment (start 180.975 54.76875) (end 180.49875 55.245) (width 0.2) (layer "F.Cu") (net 3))
 (segment (start 185.7375 83.352164) (end 185.7375 54.76875) (width 0.2) (layer "F.Cu") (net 3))
 (segment (start 180.49875 55.245) (end 167.5225 55.245) (width 0.2) (layer "F.Cu") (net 3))
 (segment (start 172.4025 90.32875) (end 178.760914 90.32875) (width 0.2) (layer "F.Cu") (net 3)))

